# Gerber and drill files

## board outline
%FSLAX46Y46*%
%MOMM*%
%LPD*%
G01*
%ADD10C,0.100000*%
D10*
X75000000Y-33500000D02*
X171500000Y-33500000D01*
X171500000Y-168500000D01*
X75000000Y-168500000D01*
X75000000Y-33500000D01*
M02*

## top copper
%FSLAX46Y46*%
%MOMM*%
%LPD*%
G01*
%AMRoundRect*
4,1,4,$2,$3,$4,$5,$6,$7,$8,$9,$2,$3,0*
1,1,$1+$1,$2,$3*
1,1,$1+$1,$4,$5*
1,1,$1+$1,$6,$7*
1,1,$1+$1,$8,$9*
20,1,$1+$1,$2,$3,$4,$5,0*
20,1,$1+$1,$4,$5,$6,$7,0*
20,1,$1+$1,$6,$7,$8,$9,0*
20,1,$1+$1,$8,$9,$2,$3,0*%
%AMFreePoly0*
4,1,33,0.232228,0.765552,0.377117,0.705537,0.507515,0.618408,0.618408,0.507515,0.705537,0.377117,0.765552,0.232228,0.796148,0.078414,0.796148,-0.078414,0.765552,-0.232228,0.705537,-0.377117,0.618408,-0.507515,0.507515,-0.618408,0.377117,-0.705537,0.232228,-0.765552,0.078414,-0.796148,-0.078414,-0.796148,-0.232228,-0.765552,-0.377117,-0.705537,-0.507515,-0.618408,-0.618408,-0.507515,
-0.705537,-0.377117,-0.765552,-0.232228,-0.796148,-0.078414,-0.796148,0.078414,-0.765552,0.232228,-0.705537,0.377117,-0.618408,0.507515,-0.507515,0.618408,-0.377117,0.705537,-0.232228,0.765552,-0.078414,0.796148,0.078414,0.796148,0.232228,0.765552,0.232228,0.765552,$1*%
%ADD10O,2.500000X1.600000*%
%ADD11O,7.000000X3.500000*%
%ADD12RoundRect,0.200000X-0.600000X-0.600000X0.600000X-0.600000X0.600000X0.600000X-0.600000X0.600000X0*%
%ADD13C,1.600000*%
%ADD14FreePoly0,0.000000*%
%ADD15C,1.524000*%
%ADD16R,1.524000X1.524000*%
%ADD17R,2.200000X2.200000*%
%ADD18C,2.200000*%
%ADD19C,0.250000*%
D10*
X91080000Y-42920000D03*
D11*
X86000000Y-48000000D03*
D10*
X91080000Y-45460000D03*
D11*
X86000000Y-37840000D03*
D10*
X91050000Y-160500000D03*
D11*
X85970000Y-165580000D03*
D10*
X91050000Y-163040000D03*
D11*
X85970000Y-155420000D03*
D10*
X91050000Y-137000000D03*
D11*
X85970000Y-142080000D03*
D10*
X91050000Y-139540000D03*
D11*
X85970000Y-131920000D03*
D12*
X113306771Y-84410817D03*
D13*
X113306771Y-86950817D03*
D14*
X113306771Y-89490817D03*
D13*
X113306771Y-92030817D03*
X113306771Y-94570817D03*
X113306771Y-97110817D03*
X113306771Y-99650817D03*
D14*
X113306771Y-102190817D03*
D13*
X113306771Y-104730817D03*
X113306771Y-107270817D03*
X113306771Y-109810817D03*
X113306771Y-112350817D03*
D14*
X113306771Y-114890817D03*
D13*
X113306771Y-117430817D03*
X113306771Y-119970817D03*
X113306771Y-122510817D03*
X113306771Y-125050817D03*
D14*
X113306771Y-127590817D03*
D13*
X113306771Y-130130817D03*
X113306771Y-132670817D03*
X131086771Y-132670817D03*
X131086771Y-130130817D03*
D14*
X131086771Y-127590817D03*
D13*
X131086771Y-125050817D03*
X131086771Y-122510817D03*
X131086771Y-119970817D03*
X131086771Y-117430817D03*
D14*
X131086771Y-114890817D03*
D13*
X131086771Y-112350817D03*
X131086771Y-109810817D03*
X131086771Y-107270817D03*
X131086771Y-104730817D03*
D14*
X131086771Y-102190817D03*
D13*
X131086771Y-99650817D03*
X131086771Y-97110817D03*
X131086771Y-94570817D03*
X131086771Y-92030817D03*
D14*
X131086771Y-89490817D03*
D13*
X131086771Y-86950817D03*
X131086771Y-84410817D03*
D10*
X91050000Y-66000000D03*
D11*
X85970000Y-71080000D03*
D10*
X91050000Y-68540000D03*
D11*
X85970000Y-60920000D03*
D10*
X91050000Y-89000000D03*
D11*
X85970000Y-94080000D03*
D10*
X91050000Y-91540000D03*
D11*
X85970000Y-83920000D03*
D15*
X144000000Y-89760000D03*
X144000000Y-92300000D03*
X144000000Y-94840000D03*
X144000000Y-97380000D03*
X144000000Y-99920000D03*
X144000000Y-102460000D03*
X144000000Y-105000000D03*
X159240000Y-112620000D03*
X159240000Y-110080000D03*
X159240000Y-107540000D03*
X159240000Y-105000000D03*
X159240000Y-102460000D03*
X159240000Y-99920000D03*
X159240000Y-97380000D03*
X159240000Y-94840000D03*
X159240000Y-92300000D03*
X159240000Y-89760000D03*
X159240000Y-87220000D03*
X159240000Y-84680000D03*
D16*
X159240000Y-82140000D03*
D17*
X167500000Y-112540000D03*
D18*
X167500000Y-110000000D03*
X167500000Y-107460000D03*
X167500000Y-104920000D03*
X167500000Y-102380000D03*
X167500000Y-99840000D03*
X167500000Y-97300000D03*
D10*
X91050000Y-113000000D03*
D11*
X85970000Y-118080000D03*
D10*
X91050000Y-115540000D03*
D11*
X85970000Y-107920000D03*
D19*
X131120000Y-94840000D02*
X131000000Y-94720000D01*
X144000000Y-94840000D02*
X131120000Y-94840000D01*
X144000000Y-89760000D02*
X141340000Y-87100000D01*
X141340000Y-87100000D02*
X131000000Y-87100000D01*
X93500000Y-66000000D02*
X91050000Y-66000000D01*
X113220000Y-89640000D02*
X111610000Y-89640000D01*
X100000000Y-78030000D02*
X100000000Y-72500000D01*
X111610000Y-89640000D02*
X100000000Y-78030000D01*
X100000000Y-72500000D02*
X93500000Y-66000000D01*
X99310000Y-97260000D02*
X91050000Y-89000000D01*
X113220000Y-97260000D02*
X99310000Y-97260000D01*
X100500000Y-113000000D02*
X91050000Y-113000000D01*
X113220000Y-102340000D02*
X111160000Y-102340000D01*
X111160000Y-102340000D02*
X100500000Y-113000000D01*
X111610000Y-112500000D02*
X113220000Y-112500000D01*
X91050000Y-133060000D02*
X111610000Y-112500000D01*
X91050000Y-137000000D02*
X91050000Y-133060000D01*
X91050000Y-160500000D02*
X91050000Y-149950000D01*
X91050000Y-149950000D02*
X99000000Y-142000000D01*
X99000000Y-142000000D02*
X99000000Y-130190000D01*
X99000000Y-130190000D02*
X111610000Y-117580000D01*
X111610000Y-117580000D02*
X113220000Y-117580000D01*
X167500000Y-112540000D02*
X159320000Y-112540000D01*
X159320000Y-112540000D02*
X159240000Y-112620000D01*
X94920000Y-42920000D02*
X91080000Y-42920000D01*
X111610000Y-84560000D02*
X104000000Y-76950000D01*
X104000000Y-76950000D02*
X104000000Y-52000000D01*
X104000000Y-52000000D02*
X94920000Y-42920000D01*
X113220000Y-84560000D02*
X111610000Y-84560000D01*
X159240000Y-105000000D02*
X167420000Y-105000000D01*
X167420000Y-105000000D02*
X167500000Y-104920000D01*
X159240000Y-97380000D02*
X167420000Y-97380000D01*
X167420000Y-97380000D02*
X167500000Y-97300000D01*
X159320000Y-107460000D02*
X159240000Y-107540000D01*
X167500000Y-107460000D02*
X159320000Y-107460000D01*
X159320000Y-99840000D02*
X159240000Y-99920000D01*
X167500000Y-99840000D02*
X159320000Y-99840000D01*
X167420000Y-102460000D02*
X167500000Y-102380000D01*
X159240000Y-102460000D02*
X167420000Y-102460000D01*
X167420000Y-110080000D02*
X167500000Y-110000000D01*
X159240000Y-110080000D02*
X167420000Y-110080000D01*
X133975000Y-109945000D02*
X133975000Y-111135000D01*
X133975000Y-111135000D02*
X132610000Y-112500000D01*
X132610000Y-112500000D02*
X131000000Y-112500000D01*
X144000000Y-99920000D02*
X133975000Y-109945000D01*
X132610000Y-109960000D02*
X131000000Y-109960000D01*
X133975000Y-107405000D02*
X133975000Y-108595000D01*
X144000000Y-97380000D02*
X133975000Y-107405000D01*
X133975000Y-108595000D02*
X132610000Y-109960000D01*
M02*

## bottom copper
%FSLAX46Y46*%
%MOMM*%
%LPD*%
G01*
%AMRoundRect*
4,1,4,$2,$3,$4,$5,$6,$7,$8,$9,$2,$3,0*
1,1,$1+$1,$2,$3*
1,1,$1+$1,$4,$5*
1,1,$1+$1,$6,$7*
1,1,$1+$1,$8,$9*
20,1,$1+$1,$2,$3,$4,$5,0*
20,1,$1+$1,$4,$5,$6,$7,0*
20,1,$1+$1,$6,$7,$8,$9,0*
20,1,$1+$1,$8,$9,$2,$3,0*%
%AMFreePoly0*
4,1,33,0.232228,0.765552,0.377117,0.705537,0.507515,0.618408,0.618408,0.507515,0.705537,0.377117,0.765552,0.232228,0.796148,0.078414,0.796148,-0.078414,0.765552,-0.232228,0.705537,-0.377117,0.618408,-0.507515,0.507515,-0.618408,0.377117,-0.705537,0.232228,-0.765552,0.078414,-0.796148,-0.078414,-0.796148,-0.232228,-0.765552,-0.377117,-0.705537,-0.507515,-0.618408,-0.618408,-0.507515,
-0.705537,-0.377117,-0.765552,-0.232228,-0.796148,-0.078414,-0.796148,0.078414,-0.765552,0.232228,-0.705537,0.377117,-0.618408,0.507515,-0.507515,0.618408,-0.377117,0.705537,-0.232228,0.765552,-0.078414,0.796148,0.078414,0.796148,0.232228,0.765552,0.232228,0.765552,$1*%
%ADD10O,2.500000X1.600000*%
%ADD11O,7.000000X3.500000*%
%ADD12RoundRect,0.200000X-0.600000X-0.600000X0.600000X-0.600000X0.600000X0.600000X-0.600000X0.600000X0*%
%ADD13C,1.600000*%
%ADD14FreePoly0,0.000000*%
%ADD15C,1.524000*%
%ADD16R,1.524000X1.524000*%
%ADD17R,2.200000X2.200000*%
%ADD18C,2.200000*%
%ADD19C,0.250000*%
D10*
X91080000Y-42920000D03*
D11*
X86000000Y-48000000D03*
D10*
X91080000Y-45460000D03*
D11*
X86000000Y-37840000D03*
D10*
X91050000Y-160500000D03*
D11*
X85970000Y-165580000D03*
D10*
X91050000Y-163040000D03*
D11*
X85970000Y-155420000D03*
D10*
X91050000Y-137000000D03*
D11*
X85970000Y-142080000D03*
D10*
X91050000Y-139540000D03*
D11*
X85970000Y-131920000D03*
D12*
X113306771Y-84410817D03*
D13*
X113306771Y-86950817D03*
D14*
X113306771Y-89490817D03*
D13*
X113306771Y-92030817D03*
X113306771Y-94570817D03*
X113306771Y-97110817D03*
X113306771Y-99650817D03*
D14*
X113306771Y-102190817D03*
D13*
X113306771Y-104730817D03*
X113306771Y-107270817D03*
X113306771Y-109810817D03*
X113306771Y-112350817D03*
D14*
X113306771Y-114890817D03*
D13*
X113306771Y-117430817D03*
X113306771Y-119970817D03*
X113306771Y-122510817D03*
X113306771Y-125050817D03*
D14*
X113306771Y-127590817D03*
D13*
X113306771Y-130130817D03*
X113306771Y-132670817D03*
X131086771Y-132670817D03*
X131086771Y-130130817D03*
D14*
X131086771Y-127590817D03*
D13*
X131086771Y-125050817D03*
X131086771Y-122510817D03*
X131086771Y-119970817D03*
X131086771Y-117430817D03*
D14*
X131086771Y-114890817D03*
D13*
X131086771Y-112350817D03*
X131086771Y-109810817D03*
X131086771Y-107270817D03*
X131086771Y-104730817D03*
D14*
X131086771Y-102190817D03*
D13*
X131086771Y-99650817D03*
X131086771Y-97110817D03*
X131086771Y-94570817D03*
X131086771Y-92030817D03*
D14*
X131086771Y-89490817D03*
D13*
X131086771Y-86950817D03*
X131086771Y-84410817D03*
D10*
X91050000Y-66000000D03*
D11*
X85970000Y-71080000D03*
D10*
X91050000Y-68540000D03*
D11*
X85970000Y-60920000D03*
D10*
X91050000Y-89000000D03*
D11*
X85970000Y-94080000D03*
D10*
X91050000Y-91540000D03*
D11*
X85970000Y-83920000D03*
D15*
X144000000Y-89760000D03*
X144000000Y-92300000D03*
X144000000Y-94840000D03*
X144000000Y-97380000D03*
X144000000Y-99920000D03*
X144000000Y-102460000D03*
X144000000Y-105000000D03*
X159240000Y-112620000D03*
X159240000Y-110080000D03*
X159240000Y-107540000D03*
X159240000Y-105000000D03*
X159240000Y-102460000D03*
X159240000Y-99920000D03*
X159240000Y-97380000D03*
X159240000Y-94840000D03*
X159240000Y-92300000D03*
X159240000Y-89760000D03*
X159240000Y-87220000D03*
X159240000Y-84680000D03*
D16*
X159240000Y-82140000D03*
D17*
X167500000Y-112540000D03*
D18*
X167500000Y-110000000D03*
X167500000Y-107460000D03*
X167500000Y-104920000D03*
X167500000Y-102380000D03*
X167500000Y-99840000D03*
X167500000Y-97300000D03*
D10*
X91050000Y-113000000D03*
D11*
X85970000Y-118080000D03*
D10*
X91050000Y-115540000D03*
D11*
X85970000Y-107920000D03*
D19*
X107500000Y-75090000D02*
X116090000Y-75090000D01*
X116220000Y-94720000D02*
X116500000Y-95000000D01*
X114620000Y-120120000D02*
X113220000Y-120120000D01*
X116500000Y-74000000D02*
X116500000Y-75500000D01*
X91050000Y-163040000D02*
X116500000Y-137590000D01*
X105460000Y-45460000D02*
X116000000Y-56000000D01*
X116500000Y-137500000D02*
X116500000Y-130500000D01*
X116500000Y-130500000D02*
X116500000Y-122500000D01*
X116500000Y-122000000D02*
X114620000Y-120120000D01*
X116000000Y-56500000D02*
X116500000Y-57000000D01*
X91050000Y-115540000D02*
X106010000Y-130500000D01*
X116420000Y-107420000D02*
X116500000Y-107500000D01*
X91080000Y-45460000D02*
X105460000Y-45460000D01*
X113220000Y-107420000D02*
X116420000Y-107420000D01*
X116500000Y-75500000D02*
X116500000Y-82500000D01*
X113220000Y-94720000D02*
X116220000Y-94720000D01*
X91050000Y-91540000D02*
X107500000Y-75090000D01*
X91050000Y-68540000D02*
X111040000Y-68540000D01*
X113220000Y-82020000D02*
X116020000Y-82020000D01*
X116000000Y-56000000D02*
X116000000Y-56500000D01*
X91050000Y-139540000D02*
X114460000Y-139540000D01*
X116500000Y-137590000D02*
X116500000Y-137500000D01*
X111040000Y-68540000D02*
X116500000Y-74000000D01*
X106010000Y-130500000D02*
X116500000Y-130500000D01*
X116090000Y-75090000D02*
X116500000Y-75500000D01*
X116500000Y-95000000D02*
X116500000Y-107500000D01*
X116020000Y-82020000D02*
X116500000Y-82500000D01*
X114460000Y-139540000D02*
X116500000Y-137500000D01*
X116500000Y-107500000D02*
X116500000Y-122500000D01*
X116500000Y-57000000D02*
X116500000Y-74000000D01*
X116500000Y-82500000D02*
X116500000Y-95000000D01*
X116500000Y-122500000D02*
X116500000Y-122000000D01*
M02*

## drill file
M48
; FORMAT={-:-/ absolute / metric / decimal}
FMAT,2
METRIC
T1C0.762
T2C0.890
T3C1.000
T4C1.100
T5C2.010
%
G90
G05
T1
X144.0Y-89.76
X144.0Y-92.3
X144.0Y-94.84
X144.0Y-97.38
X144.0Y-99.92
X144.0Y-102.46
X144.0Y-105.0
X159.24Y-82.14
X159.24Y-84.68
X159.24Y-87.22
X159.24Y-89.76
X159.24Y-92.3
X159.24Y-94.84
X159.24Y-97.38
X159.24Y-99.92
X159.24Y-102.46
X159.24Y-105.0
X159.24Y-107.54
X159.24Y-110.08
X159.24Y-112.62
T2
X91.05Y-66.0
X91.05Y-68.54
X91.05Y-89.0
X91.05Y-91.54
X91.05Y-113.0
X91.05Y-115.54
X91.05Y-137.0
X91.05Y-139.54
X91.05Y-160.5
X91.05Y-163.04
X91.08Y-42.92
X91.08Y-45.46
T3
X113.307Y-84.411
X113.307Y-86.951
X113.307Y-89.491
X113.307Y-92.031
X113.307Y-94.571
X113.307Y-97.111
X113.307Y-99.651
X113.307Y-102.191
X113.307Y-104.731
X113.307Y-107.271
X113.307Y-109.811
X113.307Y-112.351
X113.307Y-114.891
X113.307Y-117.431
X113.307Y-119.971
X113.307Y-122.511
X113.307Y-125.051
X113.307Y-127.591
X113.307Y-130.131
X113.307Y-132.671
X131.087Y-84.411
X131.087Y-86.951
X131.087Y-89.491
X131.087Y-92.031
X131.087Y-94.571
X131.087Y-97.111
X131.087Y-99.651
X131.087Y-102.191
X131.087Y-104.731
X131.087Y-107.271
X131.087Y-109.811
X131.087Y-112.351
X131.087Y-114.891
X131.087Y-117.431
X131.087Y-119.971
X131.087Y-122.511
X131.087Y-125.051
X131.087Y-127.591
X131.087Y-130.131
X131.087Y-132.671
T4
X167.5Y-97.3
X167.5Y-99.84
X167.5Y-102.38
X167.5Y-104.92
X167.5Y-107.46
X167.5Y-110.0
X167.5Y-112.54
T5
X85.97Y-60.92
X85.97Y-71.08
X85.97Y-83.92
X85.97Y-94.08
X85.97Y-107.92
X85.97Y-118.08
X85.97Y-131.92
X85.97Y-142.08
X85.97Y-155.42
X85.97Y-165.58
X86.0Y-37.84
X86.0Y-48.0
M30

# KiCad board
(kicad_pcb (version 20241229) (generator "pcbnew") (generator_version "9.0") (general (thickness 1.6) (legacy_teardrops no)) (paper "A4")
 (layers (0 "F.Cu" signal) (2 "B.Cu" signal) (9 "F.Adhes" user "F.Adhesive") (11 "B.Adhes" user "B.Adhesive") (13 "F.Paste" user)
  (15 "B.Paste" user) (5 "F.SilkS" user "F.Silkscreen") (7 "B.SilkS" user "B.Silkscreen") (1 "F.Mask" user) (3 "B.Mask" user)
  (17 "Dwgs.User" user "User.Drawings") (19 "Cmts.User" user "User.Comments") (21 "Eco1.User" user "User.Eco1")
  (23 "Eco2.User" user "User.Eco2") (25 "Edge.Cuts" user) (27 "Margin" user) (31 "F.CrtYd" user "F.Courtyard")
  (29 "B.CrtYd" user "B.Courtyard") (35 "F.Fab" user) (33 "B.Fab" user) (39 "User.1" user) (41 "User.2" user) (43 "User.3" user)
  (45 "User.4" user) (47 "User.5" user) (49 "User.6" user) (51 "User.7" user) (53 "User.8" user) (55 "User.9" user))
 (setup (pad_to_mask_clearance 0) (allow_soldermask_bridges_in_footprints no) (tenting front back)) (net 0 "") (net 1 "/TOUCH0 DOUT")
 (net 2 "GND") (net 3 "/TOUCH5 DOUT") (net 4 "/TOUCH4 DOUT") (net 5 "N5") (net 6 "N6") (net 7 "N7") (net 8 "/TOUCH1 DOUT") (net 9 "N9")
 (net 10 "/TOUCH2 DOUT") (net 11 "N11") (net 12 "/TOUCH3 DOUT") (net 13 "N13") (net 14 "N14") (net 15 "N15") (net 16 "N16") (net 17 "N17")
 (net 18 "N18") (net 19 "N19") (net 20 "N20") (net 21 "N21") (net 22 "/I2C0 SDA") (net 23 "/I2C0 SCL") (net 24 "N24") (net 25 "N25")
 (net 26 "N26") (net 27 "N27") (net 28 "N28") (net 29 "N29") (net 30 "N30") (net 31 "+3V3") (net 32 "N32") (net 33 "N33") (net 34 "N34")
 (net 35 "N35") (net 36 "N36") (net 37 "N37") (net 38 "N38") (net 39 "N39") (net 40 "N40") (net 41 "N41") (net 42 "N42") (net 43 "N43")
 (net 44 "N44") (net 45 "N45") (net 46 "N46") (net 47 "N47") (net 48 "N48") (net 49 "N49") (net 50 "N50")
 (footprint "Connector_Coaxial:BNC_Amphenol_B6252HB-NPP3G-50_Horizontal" (layer "F.Cu") (at 91.08 42.92 90)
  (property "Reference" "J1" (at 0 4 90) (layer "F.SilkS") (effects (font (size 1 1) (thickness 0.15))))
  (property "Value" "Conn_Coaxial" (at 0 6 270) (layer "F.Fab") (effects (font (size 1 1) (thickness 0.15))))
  (pad "1" thru_hole oval (at 0 0 90) (size 1.6 2.5) (drill 0.89) (layers "*.Cu" "*.Mask") (remove_unused_layers no) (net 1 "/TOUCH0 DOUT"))
  (pad "2" thru_hole oval (at -5.08 -5.08 90) (size 3.5 7) (drill 2.01) (layers "*.Cu" "*.Mask") (remove_unused_layers no) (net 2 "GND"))
  (pad "2" thru_hole oval (at -2.54 0 90) (size 1.6 2.5) (drill 0.89) (layers "*.Cu" "*.Mask") (remove_unused_layers no) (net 2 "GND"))
  (pad "2" thru_hole oval (at 5.08 -5.08 90) (size 3.5 7) (drill 2.01) (layers "*.Cu" "*.Mask") (remove_unused_layers no) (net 2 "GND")))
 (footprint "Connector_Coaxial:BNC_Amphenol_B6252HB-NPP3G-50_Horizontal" (layer "F.Cu") (at 91.05 160.5 90)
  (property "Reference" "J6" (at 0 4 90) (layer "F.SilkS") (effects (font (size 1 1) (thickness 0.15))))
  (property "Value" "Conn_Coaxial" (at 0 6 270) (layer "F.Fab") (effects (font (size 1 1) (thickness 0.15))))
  (pad "1" thru_hole oval (at 0 0 90) (size 1.6 2.5) (drill 0.89) (layers "*.Cu" "*.Mask") (remove_unused_layers no) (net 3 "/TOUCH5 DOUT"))
  (pad "2" thru_hole oval (at -5.08 -5.08 90) (size 3.5 7) (drill 2.01) (layers "*.Cu" "*.Mask") (remove_unused_layers no) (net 2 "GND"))
  (pad "2" thru_hole oval (at -2.54 0 90) (size 1.6 2.5) (drill 0.89) (layers "*.Cu" "*.Mask") (remove_unused_layers no) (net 2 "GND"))
  (pad "2" thru_hole oval (at 5.08 -5.08 90) (size 3.5 7) (drill 2.01) (layers "*.Cu" "*.Mask") (remove_unused_layers no) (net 2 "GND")))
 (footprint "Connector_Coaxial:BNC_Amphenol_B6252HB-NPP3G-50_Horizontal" (layer "F.Cu") (at 91.05 137 90)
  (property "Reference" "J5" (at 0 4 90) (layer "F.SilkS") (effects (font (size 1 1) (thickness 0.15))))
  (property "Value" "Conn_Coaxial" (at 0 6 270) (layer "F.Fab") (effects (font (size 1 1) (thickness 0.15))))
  (pad "1" thru_hole oval (at 0 0 90) (size 1.6 2.5) (drill 0.89) (layers "*.Cu" "*.Mask") (remove_unused_layers no) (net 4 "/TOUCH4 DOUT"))
  (pad "2" thru_hole oval (at -5.08 -5.08 90) (size 3.5 7) (drill 2.01) (layers "*.Cu" "*.Mask") (remove_unused_layers no) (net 2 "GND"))
  (pad "2" thru_hole oval (at -2.54 0 90) (size 1.6 2.5) (drill 0.89) (layers "*.Cu" "*.Mask") (remove_unused_layers no) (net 2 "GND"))
  (pad "2" thru_hole oval (at 5.08 -5.08 90) (size 3.5 7) (drill 2.01) (layers "*.Cu" "*.Mask") (remove_unused_layers no) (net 2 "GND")))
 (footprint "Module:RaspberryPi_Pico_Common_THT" (layer "F.Cu") (at 113.306771 84.410817)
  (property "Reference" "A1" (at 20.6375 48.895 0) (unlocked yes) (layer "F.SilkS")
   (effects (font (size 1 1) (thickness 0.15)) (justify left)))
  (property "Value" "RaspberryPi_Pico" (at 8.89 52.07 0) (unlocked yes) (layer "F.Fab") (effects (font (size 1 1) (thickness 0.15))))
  (pad "1" thru_hole roundrect (at 0 0) (size 1.6 1.6) (drill 1) (layers "*.Cu" "*.Mask") (remove_unused_layers no) (roundrect_rratio 0.125)
   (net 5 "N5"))
  (pad "2" thru_hole circle (at 0 2.54) (size 1.6 1.6) (drill 1) (layers "*.Cu" "*.Mask") (remove_unused_layers no) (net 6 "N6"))
  (pad "3" thru_hole custom (at 0 5.08) (size 1.6 1.6) (drill 1) (layers "*.Cu" "*.Mask") (remove_unused_layers no) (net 2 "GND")
   (options (clearance outline) (anchor circle)) (primitives))
  (pad "4" thru_hole circle (at 0 7.62) (size 1.6 1.6) (drill 1) (layers "*.Cu" "*.Mask") (remove_unused_layers no) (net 1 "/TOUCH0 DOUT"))
  (pad "5" thru_hole circle (at 0 10.16) (size 1.6 1.6) (drill 1) (layers "*.Cu" "*.Mask") (remove_unused_layers no) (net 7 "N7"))
  (pad "6" thru_hole circle (at 0 12.7) (size 1.6 1.6) (drill 1) (layers "*.Cu" "*.Mask") (remove_unused_layers no) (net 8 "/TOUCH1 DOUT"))
  (pad "7" thru_hole circle (at 0 15.24) (size 1.6 1.6) (drill 1) (layers "*.Cu" "*.Mask") (remove_unused_layers no) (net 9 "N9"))
  (pad "8" thru_hole custom (at 0 17.78) (size 1.6 1.6) (drill 1) (layers "*.Cu" "*.Mask") (remove_unused_layers no) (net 2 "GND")
   (options (clearance outline) (anchor circle)) (primitives))
  (pad "9" thru_hole circle (at 0 20.32) (size 1.6 1.6) (drill 1) (layers "*.Cu" "*.Mask") (remove_unused_layers no) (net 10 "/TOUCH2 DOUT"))
  (pad "10" thru_hole circle (at 0 22.86) (size 1.6 1.6) (drill 1) (layers "*.Cu" "*.Mask") (remove_unused_layers no) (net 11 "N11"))
  (pad "11" thru_hole circle (at 0 25.4) (size 1.6 1.6) (drill 1) (layers "*.Cu" "*.Mask") (remove_unused_layers no) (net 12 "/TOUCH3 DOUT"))
  (pad "12" thru_hole circle (at 0 27.94) (size 1.6 1.6) (drill 1) (layers "*.Cu" "*.Mask") (remove_unused_layers no) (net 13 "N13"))
  (pad "13" thru_hole custom (at 0 30.48) (size 1.6 1.6) (drill 1) (layers "*.Cu" "*.Mask") (remove_unused_layers no) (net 2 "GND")
   (options (clearance outline) (anchor circle)) (primitives))
  (pad "14" thru_hole circle (at 0 33.02) (size 1.6 1.6) (drill 1) (layers "*.Cu" "*.Mask") (remove_unused_layers no) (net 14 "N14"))
  (pad "15" thru_hole circle (at 0 35.56) (size 1.6 1.6) (drill 1) (layers "*.Cu" "*.Mask") (remove_unused_layers no) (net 4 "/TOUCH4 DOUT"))
  (pad "16" thru_hole circle (at 0 38.1) (size 1.6 1.6) (drill 1) (layers "*.Cu" "*.Mask") (remove_unused_layers no) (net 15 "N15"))
  (pad "17" thru_hole circle (at 0 40.64) (size 1.6 1.6) (drill 1) (layers "*.Cu" "*.Mask") (remove_unused_layers no) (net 3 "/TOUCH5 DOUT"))
  (pad "18" thru_hole custom (at 0 43.18) (size 1.6 1.6) (drill 1) (layers "*.Cu" "*.Mask") (remove_unused_layers no) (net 2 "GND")
   (options (clearance outline) (anchor circle)) (primitives))
  (pad "19" thru_hole circle (at 0 45.72) (size 1.6 1.6) (drill 1) (layers "*.Cu" "*.Mask") (remove_unused_layers no) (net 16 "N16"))
  (pad "20" thru_hole circle (at 0 48.26) (size 1.6 1.6) (drill 1) (layers "*.Cu" "*.Mask") (remove_unused_layers no) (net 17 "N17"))
  (pad "21" thru_hole circle (at 17.78 48.26) (size 1.6 1.6) (drill 1) (layers "*.Cu" "*.Mask") (remove_unused_layers no) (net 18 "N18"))
  (pad "22" thru_hole circle (at 17.78 45.72) (size 1.6 1.6) (drill 1) (layers "*.Cu" "*.Mask") (remove_unused_layers no) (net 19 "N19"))
  (pad "23" thru_hole custom (at 17.78 43.18) (size 1.6 1.6) (drill 1) (layers "*.Cu" "*.Mask") (remove_unused_layers no) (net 2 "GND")
   (options (clearance outline) (anchor circle)) (primitives))
  (pad "24" thru_hole circle (at 17.78 40.64) (size 1.6 1.6) (drill 1) (layers "*.Cu" "*.Mask") (remove_unused_layers no) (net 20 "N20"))
  (pad "25" thru_hole circle (at 17.78 38.1) (size 1.6 1.6) (drill 1) (layers "*.Cu" "*.Mask") (remove_unused_layers no) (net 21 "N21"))
  (pad "26" thru_hole circle (at 17.78 35.56) (size 1.6 1.6) (drill 1) (layers "*.Cu" "*.Mask") (remove_unused_layers no)
   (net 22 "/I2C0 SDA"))
  (pad "27" thru_hole circle (at 17.78 33.02) (size 1.6 1.6) (drill 1) (layers "*.Cu" "*.Mask") (remove_unused_layers no)
   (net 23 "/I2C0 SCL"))
  (pad "28" thru_hole custom (at 17.78 30.48) (size 1.6 1.6) (drill 1) (layers "*.Cu" "*.Mask") (remove_unused_layers no) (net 2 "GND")
   (options (clearance outline) (anchor circle)) (primitives))
  (pad "29" thru_hole circle (at 17.78 27.94) (size 1.6 1.6) (drill 1) (layers "*.Cu" "*.Mask") (remove_unused_layers no) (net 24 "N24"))
  (pad "30" thru_hole circle (at 17.78 25.4) (size 1.6 1.6) (drill 1) (layers "*.Cu" "*.Mask") (remove_unused_layers no) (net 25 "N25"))
  (pad "31" thru_hole circle (at 17.78 22.86) (size 1.6 1.6) (drill 1) (layers "*.Cu" "*.Mask") (remove_unused_layers no) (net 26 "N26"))
  (pad "32" thru_hole circle (at 17.78 20.32) (size 1.6 1.6) (drill 1) (layers "*.Cu" "*.Mask") (remove_unused_layers no) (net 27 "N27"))
  (pad "33" thru_hole custom (at 17.78 17.78) (size 1.6 1.6) (drill 1) (layers "*.Cu" "*.Mask") (remove_unused_layers no) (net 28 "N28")
   (options (clearance outline) (anchor circle)) (primitives))
  (pad "34" thru_hole circle (at 17.78 15.24) (size 1.6 1.6) (drill 1) (layers "*.Cu" "*.Mask") (remove_unused_layers no) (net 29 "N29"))
  (pad "35" thru_hole circle (at 17.78 12.7) (size 1.6 1.6) (drill 1) (layers "*.Cu" "*.Mask") (remove_unused_layers no) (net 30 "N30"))
  (pad "36" thru_hole circle (at 17.78 10.16) (size 1.6 1.6) (drill 1) (layers "*.Cu" "*.Mask") (remove_unused_layers no) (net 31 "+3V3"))
  (pad "37" thru_hole circle (at 17.78 7.62) (size 1.6 1.6) (drill 1) (layers "*.Cu" "*.Mask") (remove_unused_layers no) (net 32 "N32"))
  (pad "38" thru_hole custom (at 17.78 5.08) (size 1.6 1.6) (drill 1) (layers "*.Cu" "*.Mask") (remove_unused_layers no) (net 2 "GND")
   (options (clearance outline) (anchor circle)) (primitives))
  (pad "39" thru_hole circle (at 17.78 2.54) (size 1.6 1.6) (drill 1) (layers "*.Cu" "*.Mask") (remove_unused_layers no) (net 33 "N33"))
  (pad "40" thru_hole circle (at 17.78 0) (size 1.6 1.6) (drill 1) (layers "*.Cu" "*.Mask") (remove_unused_layers no) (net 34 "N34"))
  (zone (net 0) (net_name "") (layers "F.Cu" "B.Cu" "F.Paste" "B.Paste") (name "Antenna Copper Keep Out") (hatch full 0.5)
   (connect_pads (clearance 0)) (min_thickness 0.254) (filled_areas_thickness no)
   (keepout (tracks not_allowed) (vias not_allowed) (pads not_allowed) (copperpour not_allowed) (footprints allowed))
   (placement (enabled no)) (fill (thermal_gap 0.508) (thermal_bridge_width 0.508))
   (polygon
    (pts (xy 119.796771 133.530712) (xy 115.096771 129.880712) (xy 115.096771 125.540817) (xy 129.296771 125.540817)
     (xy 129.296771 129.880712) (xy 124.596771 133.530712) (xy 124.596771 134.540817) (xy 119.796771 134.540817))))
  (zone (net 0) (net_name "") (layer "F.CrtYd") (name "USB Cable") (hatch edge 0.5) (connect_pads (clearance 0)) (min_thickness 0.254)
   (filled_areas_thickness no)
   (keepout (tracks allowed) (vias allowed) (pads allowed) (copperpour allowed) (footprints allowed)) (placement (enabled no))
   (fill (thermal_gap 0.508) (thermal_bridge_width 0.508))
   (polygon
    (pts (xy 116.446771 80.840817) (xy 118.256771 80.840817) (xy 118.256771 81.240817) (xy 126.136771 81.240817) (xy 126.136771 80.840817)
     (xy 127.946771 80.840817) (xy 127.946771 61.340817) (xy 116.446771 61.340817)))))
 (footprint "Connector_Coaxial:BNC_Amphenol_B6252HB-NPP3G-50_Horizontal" (layer "F.Cu") (at 91.05 66 90)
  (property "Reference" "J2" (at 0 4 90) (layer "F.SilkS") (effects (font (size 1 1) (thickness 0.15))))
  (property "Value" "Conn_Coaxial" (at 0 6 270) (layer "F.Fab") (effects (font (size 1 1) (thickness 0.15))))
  (pad "1" thru_hole oval (at 0 0 90) (size 1.6 2.5) (drill 0.89) (layers "*.Cu" "*.Mask") (remove_unused_layers no) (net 8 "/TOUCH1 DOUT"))
  (pad "2" thru_hole oval (at -5.08 -5.08 90) (size 3.5 7) (drill 2.01) (layers "*.Cu" "*.Mask") (remove_unused_layers no) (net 2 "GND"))
  (pad "2" thru_hole oval (at -2.54 0 90) (size 1.6 2.5) (drill 0.89) (layers "*.Cu" "*.Mask") (remove_unused_layers no) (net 2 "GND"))
  (pad "2" thru_hole oval (at 5.08 -5.08 90) (size 3.5 7) (drill 2.01) (layers "*.Cu" "*.Mask") (remove_unused_layers no) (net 2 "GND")))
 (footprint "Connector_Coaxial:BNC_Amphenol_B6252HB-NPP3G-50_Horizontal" (layer "F.Cu") (at 91.05 89 90)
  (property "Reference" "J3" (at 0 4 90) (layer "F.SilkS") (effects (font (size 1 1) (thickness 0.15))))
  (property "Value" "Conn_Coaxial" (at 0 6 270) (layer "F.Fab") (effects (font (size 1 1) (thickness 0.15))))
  (pad "1" thru_hole oval (at 0 0 90) (size 1.6 2.5) (drill 0.89) (layers "*.Cu" "*.Mask") (remove_unused_layers no) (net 10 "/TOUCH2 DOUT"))
  (pad "2" thru_hole oval (at -5.08 -5.08 90) (size 3.5 7) (drill 2.01) (layers "*.Cu" "*.Mask") (remove_unused_layers no) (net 2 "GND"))
  (pad "2" thru_hole oval (at -2.54 0 90) (size 1.6 2.5) (drill 0.89) (layers "*.Cu" "*.Mask") (remove_unused_layers no) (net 2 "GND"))
  (pad "2" thru_hole oval (at 5.08 -5.08 90) (size 3.5 7) (drill 2.01) (layers "*.Cu" "*.Mask") (remove_unused_layers no) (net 2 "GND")))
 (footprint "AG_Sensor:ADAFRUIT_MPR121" (layer "F.Cu") (at 152.89 94.84 -90)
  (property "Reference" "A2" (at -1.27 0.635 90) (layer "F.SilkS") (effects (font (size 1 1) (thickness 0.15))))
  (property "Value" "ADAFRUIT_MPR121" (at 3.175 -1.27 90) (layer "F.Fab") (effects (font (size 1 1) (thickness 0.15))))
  (pad "1" thru_hole circle (at -5.08 8.89 270) (size 1.524 1.524) (drill 0.762) (layers "*.Cu" "*.Mask") (remove_unused_layers no)
   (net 31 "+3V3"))
  (pad "2" thru_hole circle (at -2.54 8.89 270) (size 1.524 1.524) (drill 0.762) (layers "*.Cu" "*.Mask") (remove_unused_layers no)
   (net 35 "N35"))
  (pad "3" thru_hole circle (at 0 8.89 270) (size 1.524 1.524) (drill 0.762) (layers "*.Cu" "*.Mask") (remove_unused_layers no)
   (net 2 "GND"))
  (pad "4" thru_hole circle (at 2.54 8.89 270) (size 1.524 1.524) (drill 0.762) (layers "*.Cu" "*.Mask") (remove_unused_layers no)
   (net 23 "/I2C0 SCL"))
  (pad "5" thru_hole circle (at 5.08 8.89 270) (size 1.524 1.524) (drill 0.762) (layers "*.Cu" "*.Mask") (remove_unused_layers no)
   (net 22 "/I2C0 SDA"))
  (pad "6" thru_hole circle (at 7.62 8.89 270) (size 1.524 1.524) (drill 0.762) (layers "*.Cu" "*.Mask") (remove_unused_layers no)
   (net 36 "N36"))
  (pad "7" thru_hole circle (at 10.16 8.89 270) (size 1.524 1.524) (drill 0.762) (layers "*.Cu" "*.Mask") (remove_unused_layers no)
   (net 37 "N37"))
  (pad "8" thru_hole circle (at 17.78 -6.35 270) (size 1.524 1.524) (drill 0.762) (layers "*.Cu" "*.Mask") (remove_unused_layers no)
   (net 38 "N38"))
  (pad "9" thru_hole circle (at 15.24 -6.35 270) (size 1.524 1.524) (drill 0.762) (layers "*.Cu" "*.Mask") (remove_unused_layers no)
   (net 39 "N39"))
  (pad "10" thru_hole circle (at 12.7 -6.35 270) (size 1.524 1.524) (drill 0.762) (layers "*.Cu" "*.Mask") (remove_unused_layers no)
   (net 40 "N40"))
  (pad "11" thru_hole circle (at 10.16 -6.35) (size 1.524 1.524) (drill 0.762) (layers "*.Cu" "*.Mask") (remove_unused_layers no)
   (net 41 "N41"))
  (pad "12" thru_hole circle (at 7.62 -6.35 270) (size 1.524 1.524) (drill 0.762) (layers "*.Cu" "*.Mask") (remove_unused_layers no)
   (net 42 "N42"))
  (pad "13" thru_hole circle (at 5.08 -6.35 270) (size 1.524 1.524) (drill 0.762) (layers "*.Cu" "*.Mask") (remove_unused_layers no)
   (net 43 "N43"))
  (pad "14" thru_hole circle (at 2.54 -6.35 270) (size 1.524 1.524) (drill 0.762) (layers "*.Cu" "*.Mask") (remove_unused_layers no)
   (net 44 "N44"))
  (pad "15" thru_hole circle (at 0 -6.35 270) (size 1.524 1.524) (drill 0.762) (layers "*.Cu" "*.Mask") (remove_unused_layers no)
   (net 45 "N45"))
  (pad "16" thru_hole circle (at -2.54 -6.35 270) (size 1.524 1.524) (drill 0.762) (layers "*.Cu" "*.Mask") (remove_unused_layers no)
   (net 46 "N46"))
  (pad "17" thru_hole circle (at -5.08 -6.35 270) (size 1.524 1.524) (drill 0.762) (layers "*.Cu" "*.Mask") (remove_unused_layers no)
   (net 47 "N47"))
  (pad "18" thru_hole circle (at -7.62 -6.35 270) (size 1.524 1.524) (drill 0.762) (layers "*.Cu" "*.Mask") (remove_unused_layers no)
   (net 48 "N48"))
  (pad "19" thru_hole circle (at -10.16 -6.35 270) (size 1.524 1.524) (drill 0.762) (layers "*.Cu" "*.Mask") (remove_unused_layers no)
   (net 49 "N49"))
  (pad "20" thru_hole rect (at -12.7 -6.35 270) (size 1.524 1.524) (drill 0.762) (layers "*.Cu" "*.Mask") (remove_unused_layers no)
   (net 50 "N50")))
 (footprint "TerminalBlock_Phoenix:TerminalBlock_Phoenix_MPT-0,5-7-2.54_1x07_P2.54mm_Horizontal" (layer "F.Cu") (at 167.5 112.54 90)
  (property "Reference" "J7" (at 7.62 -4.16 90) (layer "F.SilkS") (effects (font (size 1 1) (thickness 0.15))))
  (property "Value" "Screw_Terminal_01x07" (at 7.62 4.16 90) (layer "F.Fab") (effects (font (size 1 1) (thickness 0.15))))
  (pad "1" thru_hole rect (at 0 0 90) (size 2.2 2.2) (drill 1.1) (layers "*.Cu" "*.Mask") (remove_unused_layers no) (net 38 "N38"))
  (pad "2" thru_hole circle (at 2.54 0 90) (size 2.2 2.2) (drill 1.1) (layers "*.Cu" "*.Mask") (remove_unused_layers no) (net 39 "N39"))
  (pad "3" thru_hole circle (at 5.08 0 90) (size 2.2 2.2) (drill 1.1) (layers "*.Cu" "*.Mask") (remove_unused_layers no) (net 40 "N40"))
  (pad "4" thru_hole circle (at 7.62 0 90) (size 2.2 2.2) (drill 1.1) (layers "*.Cu" "*.Mask") (remove_unused_layers no) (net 41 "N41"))
  (pad "5" thru_hole circle (at 10.16 0 90) (size 2.2 2.2) (drill 1.1) (layers "*.Cu" "*.Mask") (remove_unused_layers no) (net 42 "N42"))
  (pad "6" thru_hole circle (at 12.7 0 90) (size 2.2 2.2) (drill 1.1) (layers "*.Cu" "*.Mask") (remove_unused_layers no) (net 43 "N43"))
  (pad "7" thru_hole circle (at 15.24 0 90) (size 2.2 2.2) (drill 1.1) (layers "*.Cu" "*.Mask") (remove_unused_layers no) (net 44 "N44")))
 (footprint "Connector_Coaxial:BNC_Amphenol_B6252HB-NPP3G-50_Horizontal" (layer "F.Cu") (at 91.05 113 90)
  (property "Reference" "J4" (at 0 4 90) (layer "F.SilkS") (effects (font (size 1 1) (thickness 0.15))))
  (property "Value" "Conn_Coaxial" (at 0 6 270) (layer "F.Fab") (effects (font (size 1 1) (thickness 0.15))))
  (pad "1" thru_hole oval (at 0 0 90) (size 1.6 2.5) (drill 0.89) (layers "*.Cu" "*.Mask") (remove_unused_layers no) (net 12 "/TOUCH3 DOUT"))
  (pad "2" thru_hole oval (at -5.08 -5.08 90) (size 3.5 7) (drill 2.01) (layers "*.Cu" "*.Mask") (remove_unused_layers no) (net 2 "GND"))
  (pad "2" thru_hole oval (at -2.54 0 90) (size 1.6 2.5) (drill 0.89) (layers "*.Cu" "*.Mask") (remove_unused_layers no) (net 2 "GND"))
  (pad "2" thru_hole oval (at 5.08 -5.08 90) (size 3.5 7) (drill 2.01) (layers "*.Cu" "*.Mask") (remove_unused_layers no) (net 2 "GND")))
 (gr_rect (start 75 33.5) (end 171.5 168.5) (stroke (width 0.1) (type default)) (fill no) (layer "Edge.Cuts"))
 (segment (start 131.12 94.84) (end 131 94.72) (width 0.25) (layer "F.Cu") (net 2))
 (segment (start 144 94.84) (end 131.12 94.84) (width 0.25) (layer "F.Cu") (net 2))
 (segment (start 107.5 75.09) (end 116.09 75.09) (width 0.25) (layer "B.Cu") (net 2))
 (segment (start 116.22 94.72) (end 116.5 95) (width 0.25) (layer "B.Cu") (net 2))
 (segment (start 114.62 120.12) (end 113.22 120.12) (width 0.25) (layer "B.Cu") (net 2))
 (segment (start 116.5 74) (end 116.5 75.5) (width 0.25) (layer "B.Cu") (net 2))
 (segment (start 91.05 163.04) (end 116.5 137.59) (width 0.25) (layer "B.Cu") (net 2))
 (segment (start 105.46 45.46) (end 116 56) (width 0.25) (layer "B.Cu") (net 2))
 (segment (start 116.5 137.5) (end 116.5 130.5) (width 0.25) (layer "B.Cu") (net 2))
 (segment (start 116.5 130.5) (end 116.5 122.5) (width 0.25) (layer "B.Cu") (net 2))
 (segment (start 116.5 122) (end 114.62 120.12) (width 0.25) (layer "B.Cu") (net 2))
 (segment (start 116 56.5) (end 116.5 57) (width 0.25) (layer "B.Cu") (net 2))
 (segment (start 91.05 115.54) (end 106.01 130.5) (width 0.25) (layer "B.Cu") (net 2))
 (segment (start 116.42 107.42) (end 116.5 107.5) (width 0.25) (layer "B.Cu") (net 2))
 (segment (start 91.08 45.46) (end 105.46 45.46) (width 0.25) (layer "B.Cu") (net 2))
 (segment (start 113.22 107.42) (end 116.42 107.42) (width 0.25) (layer "B.Cu") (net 2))
 (segment (start 116.5 75.5) (end 116.5 82.5) (width 0.25) (layer "B.Cu") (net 2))
 (segment (start 113.22 94.72) (end 116.22 94.72) (width 0.25) (layer "B.Cu") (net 2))
 (segment (start 91.05 91.54) (end 107.5 75.09) (width 0.25) (layer "B.Cu") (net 2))
 (segment (start 91.05 68.54) (end 111.04 68.54) (width 0.25) (layer "B.Cu") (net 2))
 (segment (start 113.22 82.02) (end 116.02 82.02) (width 0.25) (layer "B.Cu") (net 2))
 (segment (start 116 56) (end 116 56.5) (width 0.25) (layer "B.Cu") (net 2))
 (segment (start 91.05 139.54) (end 114.46 139.54) (width 0.25) (layer "B.Cu") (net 2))
 (segment (start 116.5 137.59) (end 116.5 137.5) (width 0.25) (layer "B.Cu") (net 2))
 (segment (start 111.04 68.54) (end 116.5 74) (width 0.25) (layer "B.Cu") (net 2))
 (segment (start 106.01 130.5) (end 116.5 130.5) (width 0.25) (layer "B.Cu") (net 2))
 (segment (start 116.09 75.09) (end 116.5 75.5) (width 0.25) (layer "B.Cu") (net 2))
 (segment (start 116.5 95) (end 116.5 107.5) (width 0.25) (layer "B.Cu") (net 2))
 (segment (start 116.02 82.02) (end 116.5 82.5) (width 0.25) (layer "B.Cu") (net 2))
 (segment (start 114.46 139.54) (end 116.5 137.5) (width 0.25) (layer "B.Cu") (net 2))
 (segment (start 116.5 107.5) (end 116.5 122.5) (width 0.25) (layer "B.Cu") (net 2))
 (segment (start 116.5 57) (end 116.5 74) (width 0.25) (layer "B.Cu") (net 2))
 (segment (start 116.5 82.5) (end 116.5 95) (width 0.25) (layer "B.Cu") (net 2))
 (segment (start 116.5 122.5) (end 116.5 122) (width 0.25) (layer "B.Cu") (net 2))
 (segment (start 144 89.76) (end 141.34 87.1) (width 0.25) (layer "F.Cu") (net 31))
 (segment (start 141.34 87.1) (end 131 87.1) (width 0.25) (layer "F.Cu") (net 31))
 (segment (start 93.5 66) (end 91.05 66) (width 0.25) (layer "F.Cu") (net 8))
 (segment (start 113.22 89.64) (end 111.61 89.64) (width 0.25) (layer "F.Cu") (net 8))
 (segment (start 100 78.03) (end 100 72.5) (width 0.25) (layer "F.Cu") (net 8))
 (segment (start 111.61 89.64) (end 100 78.03) (width 0.25) (layer "F.Cu") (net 8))
 (segment (start 100 72.5) (end 93.5 66) (width 0.25) (layer "F.Cu") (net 8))
 (segment (start 99.31 97.26) (end 91.05 89) (width 0.25) (layer "F.Cu") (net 10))
 (segment (start 113.22 97.26) (end 99.31 97.26) (width 0.25) (layer "F.Cu") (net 10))
 (segment (start 100.5 113) (end 91.05 113) (width 0.25) (layer "F.Cu") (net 12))
 (segment (start 113.22 102.34) (end 111.16 102.34) (width 0.25) (layer "F.Cu") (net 12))
 (segment (start 111.16 102.34) (end 100.5 113) (width 0.25) (layer "F.Cu") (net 12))
 (segment (start 111.61 112.5) (end 113.22 112.5) (width 0.25) (layer "F.Cu") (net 4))
 (segment (start 91.05 133.06) (end 111.61 112.5) (width 0.25) (layer "F.Cu") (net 4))
 (segment (start 91.05 137) (end 91.05 133.06) (width 0.25) (layer "F.Cu") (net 4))
 (segment (start 91.05 160.5) (end 91.05 149.95) (width 0.25) (layer "F.Cu") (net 3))
 (segment (start 91.05 149.95) (end 99 142) (width 0.25) (layer "F.Cu") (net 3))
 (segment (start 99 142) (end 99 130.19) (width 0.25) (layer "F.Cu") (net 3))
 (segment (start 99 130.19) (end 111.61 117.58) (width 0.25) (layer "F.Cu") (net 3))
 (segment (start 111.61 117.58) (end 113.22 117.58) (width 0.25) (layer "F.Cu") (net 3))
 (segment (start 167.5 112.54) (end 159.32 112.54) (width 0.25) (layer "F.Cu") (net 38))
 (segment (start 159.32 112.54) (end 159.24 112.62) (width 0.25) (layer "F.Cu") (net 38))
 (segment (start 94.92 42.92) (end 91.08 42.92) (width 0.25) (layer "F.Cu") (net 1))
 (segment (start 111.61 84.56) (end 104 76.95) (width 0.25) (layer "F.Cu") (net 1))
 (segment (start 104 76.95) (end 104 52) (width 0.25) (layer "F.Cu") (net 1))
 (segment (start 104 52) (end 94.92 42.92) (width 0.25) (layer "F.Cu") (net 1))
 (segment (start 113.22 84.56) (end 111.61 84.56) (width 0.25) (layer "F.Cu") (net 1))
 (segment (start 159.24 105) (end 167.42 105) (width 0.25) (layer "F.Cu") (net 41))
 (segment (start 167.42 105) (end 167.5 104.92) (width 0.25) (layer "F.Cu") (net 41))
 (segment (start 159.24 97.38) (end 167.42 97.38) (width 0.25) (layer "F.Cu") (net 44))
 (segment (start 167.42 97.38) (end 167.5 97.3) (width 0.25) (layer "F.Cu") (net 44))
 (segment (start 159.32 107.46) (end 159.24 107.54) (width 0.25) (layer "F.Cu") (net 40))
 (segment (start 167.5 107.46) (end 159.32 107.46) (width 0.25) (layer "F.Cu") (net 40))
 (segment (start 159.32 99.84) (end 159.24 99.92) (width 0.25) (layer "F.Cu") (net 43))
 (segment (start 167.5 99.84) (end 159.32 99.84) (width 0.25) (layer "F.Cu") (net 43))
 (segment (start 167.42 102.46) (end 167.5 102.38) (width 0.25) (layer "F.Cu") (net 42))
 (segment (start 159.24 102.46) (end 167.42 102.46) (width 0.25) (layer "F.Cu") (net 42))
 (segment (start 167.42 110.08) (end 167.5 110) (width 0.25) (layer "F.Cu") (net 39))
 (segment (start 159.24 110.08) (end 167.42 110.08) (width 0.25) (layer "F.Cu") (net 39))
 (segment (start 133.975 109.945) (end 133.975 111.135) (width 0.25) (layer "F.Cu") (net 22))
 (segment (start 133.975 111.135) (end 132.61 112.5) (width 0.25) (layer "F.Cu") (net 22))
 (segment (start 132.61 112.5) (end 131 112.5) (width 0.25) (layer "F.Cu") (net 22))
 (segment (start 144 99.92) (end 133.975 109.945) (width 0.25) (layer "F.Cu") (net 22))
 (segment (start 132.61 109.96) (end 131 109.96) (width 0.25) (layer "F.Cu") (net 23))
 (segment (start 133.975 107.405) (end 133.975 108.595) (width 0.25) (layer "F.Cu") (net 23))
 (segment (start 144 97.38) (end 133.975 107.405) (width 0.25) (layer "F.Cu") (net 23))
 (segment (start 133.975 108.595) (end 132.61 109.96) (width 0.25) (layer "F.Cu") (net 23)))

